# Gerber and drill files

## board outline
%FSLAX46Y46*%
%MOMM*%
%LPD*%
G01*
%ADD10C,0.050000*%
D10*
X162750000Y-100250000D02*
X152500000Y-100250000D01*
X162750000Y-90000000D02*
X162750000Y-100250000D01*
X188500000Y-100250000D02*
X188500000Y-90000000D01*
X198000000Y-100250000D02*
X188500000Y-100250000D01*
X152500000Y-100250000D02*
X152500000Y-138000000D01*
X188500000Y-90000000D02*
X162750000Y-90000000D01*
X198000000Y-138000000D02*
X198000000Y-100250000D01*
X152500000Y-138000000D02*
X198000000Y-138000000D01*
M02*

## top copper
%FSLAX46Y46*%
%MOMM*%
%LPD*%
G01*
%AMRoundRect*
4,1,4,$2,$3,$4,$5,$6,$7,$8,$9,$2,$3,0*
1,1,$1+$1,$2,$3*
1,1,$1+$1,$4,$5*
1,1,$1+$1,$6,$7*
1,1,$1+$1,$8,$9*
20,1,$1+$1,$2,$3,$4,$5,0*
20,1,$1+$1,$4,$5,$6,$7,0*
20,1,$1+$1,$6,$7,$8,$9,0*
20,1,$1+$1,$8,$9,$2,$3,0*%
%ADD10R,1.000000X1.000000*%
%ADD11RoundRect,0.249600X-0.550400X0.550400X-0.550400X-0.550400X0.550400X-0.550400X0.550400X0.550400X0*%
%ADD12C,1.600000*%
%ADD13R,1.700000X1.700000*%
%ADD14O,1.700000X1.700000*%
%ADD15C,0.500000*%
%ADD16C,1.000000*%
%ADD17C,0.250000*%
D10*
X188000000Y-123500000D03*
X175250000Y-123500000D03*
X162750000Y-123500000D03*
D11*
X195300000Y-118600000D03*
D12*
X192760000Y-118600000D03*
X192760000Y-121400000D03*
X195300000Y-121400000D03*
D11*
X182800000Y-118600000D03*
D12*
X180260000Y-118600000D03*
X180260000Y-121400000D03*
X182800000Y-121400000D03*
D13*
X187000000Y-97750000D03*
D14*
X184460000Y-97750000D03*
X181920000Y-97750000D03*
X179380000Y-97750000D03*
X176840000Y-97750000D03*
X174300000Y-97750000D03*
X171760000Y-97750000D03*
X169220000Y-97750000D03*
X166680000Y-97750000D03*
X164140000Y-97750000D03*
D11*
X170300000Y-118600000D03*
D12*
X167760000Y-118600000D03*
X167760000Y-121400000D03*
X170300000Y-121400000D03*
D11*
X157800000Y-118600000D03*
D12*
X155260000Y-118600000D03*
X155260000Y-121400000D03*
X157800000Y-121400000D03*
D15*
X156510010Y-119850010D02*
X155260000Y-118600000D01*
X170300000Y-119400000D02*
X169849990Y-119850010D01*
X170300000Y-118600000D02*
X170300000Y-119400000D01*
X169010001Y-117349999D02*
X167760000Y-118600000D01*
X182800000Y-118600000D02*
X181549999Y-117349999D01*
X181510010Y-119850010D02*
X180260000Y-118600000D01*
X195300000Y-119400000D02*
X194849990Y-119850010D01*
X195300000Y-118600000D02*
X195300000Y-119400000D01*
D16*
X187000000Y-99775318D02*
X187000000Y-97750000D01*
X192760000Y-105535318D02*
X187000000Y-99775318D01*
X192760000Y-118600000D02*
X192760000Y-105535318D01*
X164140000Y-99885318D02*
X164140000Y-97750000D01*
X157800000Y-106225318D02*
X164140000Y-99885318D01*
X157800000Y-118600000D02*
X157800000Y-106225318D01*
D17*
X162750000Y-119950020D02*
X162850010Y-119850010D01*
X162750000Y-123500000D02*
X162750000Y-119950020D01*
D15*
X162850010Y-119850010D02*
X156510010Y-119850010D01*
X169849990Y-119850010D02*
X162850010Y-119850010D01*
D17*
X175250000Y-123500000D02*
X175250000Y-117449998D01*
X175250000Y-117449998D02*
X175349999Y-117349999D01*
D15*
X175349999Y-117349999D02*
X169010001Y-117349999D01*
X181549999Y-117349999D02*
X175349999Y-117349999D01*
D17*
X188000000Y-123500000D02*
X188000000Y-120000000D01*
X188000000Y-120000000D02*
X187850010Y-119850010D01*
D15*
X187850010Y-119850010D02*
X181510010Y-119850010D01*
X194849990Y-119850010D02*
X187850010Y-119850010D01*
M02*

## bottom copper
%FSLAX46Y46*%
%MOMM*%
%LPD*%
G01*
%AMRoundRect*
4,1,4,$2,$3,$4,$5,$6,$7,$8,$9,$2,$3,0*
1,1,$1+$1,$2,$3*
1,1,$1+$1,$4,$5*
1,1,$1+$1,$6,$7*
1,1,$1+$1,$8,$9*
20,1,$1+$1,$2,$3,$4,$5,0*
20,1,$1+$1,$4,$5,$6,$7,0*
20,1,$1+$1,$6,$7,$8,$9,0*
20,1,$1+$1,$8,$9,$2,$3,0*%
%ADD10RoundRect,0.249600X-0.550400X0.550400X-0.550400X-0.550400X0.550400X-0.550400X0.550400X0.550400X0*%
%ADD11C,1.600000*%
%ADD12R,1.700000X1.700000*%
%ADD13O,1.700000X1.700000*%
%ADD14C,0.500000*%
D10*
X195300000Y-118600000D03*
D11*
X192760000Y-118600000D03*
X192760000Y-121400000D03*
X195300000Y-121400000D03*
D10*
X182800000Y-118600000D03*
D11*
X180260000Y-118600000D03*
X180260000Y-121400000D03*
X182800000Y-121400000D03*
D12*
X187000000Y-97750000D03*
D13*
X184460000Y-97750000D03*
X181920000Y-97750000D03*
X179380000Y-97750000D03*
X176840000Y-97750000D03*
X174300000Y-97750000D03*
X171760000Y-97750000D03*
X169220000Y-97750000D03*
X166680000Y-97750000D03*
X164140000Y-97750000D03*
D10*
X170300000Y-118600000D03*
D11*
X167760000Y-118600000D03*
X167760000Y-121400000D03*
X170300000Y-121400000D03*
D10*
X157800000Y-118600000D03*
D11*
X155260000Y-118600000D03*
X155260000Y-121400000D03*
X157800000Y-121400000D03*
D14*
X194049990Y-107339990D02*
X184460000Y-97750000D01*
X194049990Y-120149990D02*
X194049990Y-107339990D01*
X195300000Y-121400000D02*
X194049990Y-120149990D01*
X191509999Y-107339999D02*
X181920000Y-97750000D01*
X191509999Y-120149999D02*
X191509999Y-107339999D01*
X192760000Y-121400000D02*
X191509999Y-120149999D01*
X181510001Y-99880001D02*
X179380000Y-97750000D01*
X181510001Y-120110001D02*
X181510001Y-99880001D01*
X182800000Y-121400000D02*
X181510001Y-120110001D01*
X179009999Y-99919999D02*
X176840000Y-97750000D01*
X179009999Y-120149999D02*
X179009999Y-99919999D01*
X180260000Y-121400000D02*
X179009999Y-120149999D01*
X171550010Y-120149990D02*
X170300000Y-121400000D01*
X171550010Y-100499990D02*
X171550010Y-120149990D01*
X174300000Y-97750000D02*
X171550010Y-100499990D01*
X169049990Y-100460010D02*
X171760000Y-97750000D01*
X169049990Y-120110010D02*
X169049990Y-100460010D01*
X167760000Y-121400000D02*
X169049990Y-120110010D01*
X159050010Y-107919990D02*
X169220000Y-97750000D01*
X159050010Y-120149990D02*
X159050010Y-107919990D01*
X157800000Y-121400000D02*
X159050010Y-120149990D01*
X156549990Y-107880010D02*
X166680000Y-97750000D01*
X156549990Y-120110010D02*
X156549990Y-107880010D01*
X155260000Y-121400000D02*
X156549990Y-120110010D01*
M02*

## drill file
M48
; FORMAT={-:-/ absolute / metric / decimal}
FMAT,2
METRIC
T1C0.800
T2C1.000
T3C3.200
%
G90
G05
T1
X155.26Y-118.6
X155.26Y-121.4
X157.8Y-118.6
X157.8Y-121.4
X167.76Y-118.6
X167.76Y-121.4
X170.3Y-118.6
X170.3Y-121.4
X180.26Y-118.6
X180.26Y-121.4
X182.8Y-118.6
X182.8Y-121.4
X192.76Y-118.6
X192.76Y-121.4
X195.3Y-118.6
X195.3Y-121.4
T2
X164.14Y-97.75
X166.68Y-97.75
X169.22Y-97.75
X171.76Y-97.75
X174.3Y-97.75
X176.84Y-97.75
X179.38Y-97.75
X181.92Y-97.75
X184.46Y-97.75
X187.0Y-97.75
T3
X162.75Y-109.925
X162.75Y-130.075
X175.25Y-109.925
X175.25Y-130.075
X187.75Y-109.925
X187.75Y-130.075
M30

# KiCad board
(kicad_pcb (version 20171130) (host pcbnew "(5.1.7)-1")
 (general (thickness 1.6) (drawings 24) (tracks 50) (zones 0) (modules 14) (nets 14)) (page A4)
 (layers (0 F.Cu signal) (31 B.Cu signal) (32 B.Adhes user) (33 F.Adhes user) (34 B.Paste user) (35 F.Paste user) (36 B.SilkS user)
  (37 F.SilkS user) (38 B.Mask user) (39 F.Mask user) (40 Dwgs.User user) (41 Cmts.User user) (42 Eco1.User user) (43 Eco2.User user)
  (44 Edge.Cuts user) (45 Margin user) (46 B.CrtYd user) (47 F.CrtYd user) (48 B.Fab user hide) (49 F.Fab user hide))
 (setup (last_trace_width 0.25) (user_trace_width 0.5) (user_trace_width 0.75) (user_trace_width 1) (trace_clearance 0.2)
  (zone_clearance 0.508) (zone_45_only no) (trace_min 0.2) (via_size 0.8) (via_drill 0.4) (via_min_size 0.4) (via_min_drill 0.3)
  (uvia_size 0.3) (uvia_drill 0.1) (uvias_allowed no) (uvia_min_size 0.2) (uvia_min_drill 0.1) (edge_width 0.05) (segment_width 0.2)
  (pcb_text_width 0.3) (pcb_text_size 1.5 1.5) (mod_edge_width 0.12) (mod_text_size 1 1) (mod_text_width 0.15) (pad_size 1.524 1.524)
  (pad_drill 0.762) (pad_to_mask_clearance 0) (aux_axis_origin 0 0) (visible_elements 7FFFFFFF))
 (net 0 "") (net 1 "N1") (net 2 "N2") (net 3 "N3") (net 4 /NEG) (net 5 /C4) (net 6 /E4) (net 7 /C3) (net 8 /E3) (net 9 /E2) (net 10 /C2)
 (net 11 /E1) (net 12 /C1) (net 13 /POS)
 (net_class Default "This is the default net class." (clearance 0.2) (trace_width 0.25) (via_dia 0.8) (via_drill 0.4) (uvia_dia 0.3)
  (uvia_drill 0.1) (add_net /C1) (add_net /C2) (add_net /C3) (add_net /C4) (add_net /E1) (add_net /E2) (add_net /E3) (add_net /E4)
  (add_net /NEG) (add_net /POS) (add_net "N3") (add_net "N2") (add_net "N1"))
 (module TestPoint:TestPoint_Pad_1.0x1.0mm (layer F.Cu) (at 188 123.5)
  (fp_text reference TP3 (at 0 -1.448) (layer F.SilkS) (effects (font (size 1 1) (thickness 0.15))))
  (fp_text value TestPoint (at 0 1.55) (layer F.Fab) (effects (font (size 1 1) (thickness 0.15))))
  (pad 1 smd rect (at 0 0) (size 1 1) (layers F.Cu F.Mask) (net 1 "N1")))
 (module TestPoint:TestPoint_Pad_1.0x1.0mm (layer F.Cu) (at 175.25 123.5)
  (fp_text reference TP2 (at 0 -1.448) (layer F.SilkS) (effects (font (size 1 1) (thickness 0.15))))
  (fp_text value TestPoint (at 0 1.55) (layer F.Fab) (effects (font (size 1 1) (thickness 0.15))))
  (pad 1 smd rect (at 0 0) (size 1 1) (layers F.Cu F.Mask) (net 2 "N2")))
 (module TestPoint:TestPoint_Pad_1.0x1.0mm (layer F.Cu) (at 162.75 123.5)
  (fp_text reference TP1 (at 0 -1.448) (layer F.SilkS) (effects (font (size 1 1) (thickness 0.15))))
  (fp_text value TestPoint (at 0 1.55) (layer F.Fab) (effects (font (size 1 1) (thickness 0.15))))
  (pad 1 smd rect (at 0 0) (size 1 1) (layers F.Cu F.Mask) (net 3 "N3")))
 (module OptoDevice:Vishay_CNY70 (layer F.Cu) (at 195.3 118.6 270)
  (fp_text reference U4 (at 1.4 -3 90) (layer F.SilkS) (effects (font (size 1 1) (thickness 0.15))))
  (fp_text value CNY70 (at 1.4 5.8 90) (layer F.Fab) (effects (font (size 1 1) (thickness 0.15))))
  (pad 1 thru_hole roundrect (at 0 0 270) (size 1.6 1.6) (drill 0.8) (layers *.Cu *.Mask) (roundrect_rratio 0.156) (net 1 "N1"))
  (pad 2 thru_hole circle (at 0 2.54 270) (size 1.6 1.6) (drill 0.8) (layers *.Cu *.Mask) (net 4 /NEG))
  (pad 3 thru_hole circle (at 2.8 2.54 270) (size 1.6 1.6) (drill 0.8) (layers *.Cu *.Mask) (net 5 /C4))
  (pad 4 thru_hole circle (at 2.8 0 270) (size 1.6 1.6) (drill 0.8) (layers *.Cu *.Mask) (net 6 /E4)))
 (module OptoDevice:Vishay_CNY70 (layer F.Cu) (at 182.8 118.6 270)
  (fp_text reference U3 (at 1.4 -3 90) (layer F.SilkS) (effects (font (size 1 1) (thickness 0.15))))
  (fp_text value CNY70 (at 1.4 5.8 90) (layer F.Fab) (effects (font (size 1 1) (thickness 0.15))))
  (pad 1 thru_hole roundrect (at 0 0 270) (size 1.6 1.6) (drill 0.8) (layers *.Cu *.Mask) (roundrect_rratio 0.156) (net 2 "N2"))
  (pad 2 thru_hole circle (at 0 2.54 270) (size 1.6 1.6) (drill 0.8) (layers *.Cu *.Mask) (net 1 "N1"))
  (pad 3 thru_hole circle (at 2.8 2.54 270) (size 1.6 1.6) (drill 0.8) (layers *.Cu *.Mask) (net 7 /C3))
  (pad 4 thru_hole circle (at 2.8 0 270) (size 1.6 1.6) (drill 0.8) (layers *.Cu *.Mask) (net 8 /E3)))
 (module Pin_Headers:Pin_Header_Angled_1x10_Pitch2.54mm (layer B.Cu) (at 187 97.75 90)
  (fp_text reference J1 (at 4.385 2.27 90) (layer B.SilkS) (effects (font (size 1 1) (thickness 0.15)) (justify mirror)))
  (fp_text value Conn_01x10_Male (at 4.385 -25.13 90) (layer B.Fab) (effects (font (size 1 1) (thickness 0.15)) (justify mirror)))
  (pad 1 thru_hole rect (at 0 0 90) (size 1.7 1.7) (drill 1) (layers *.Cu *.Mask) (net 4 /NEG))
  (pad 2 thru_hole oval (at 0 -2.54 90) (size 1.7 1.7) (drill 1) (layers *.Cu *.Mask) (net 6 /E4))
  (pad 3 thru_hole oval (at 0 -5.08 90) (size 1.7 1.7) (drill 1) (layers *.Cu *.Mask) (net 5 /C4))
  (pad 4 thru_hole oval (at 0 -7.62 90) (size 1.7 1.7) (drill 1) (layers *.Cu *.Mask) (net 8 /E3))
  (pad 5 thru_hole oval (at 0 -10.16 90) (size 1.7 1.7) (drill 1) (layers *.Cu *.Mask) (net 7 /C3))
  (pad 6 thru_hole oval (at 0 -12.7 90) (size 1.7 1.7) (drill 1) (layers *.Cu *.Mask) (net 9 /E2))
  (pad 7 thru_hole oval (at 0 -15.24 90) (size 1.7 1.7) (drill 1) (layers *.Cu *.Mask) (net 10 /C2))
  (pad 8 thru_hole oval (at 0 -17.78 90) (size 1.7 1.7) (drill 1) (layers *.Cu *.Mask) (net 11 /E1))
  (pad 9 thru_hole oval (at 0 -20.32 90) (size 1.7 1.7) (drill 1) (layers *.Cu *.Mask) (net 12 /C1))
  (pad 10 thru_hole oval (at 0 -22.86 90) (size 1.7 1.7) (drill 1) (layers *.Cu *.Mask) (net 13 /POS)))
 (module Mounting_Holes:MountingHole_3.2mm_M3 (layer F.Cu) (at 187.75 109.925)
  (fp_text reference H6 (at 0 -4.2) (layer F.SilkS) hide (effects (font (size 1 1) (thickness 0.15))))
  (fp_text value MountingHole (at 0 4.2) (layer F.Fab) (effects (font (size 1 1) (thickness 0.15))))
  (pad 1 np_thru_hole circle (at 0 0) (size 3.2 3.2) (drill 3.2) (layers *.Cu *.Mask)))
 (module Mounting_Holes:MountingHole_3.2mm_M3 (layer F.Cu) (at 187.75 130.075)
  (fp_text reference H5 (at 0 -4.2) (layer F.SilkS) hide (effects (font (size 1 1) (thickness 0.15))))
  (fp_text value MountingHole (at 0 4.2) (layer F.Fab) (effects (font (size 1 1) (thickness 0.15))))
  (pad 1 np_thru_hole circle (at 0 0) (size 3.2 3.2) (drill 3.2) (layers *.Cu *.Mask)))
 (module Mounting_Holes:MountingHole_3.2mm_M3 (layer F.Cu) (at 175.25 109.925)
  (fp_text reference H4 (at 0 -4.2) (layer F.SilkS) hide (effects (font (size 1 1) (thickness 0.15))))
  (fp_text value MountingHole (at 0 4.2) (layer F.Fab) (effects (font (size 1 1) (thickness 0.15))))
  (pad 1 np_thru_hole circle (at 0 0) (size 3.2 3.2) (drill 3.2) (layers *.Cu *.Mask)))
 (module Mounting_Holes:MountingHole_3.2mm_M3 (layer F.Cu) (at 175.25 130.075)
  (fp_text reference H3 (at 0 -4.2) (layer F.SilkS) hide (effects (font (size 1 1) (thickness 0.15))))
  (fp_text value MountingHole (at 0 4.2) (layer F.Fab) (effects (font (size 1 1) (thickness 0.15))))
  (pad 1 np_thru_hole circle (at 0 0) (size 3.2 3.2) (drill 3.2) (layers *.Cu *.Mask)))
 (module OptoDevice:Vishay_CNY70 (layer F.Cu) (at 170.3 118.6 270)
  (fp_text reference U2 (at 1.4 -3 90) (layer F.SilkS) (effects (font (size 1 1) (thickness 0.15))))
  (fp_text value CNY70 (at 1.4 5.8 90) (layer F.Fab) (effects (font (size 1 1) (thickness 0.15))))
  (pad 1 thru_hole roundrect (at 0 0 270) (size 1.6 1.6) (drill 0.8) (layers *.Cu *.Mask) (roundrect_rratio 0.156) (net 3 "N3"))
  (pad 2 thru_hole circle (at 0 2.54 270) (size 1.6 1.6) (drill 0.8) (layers *.Cu *.Mask) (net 2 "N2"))
  (pad 3 thru_hole circle (at 2.8 2.54 270) (size 1.6 1.6) (drill 0.8) (layers *.Cu *.Mask) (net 10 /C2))
  (pad 4 thru_hole circle (at 2.8 0 270) (size 1.6 1.6) (drill 0.8) (layers *.Cu *.Mask) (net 9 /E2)))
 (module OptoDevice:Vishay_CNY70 (layer F.Cu) (at 157.8 118.6 270)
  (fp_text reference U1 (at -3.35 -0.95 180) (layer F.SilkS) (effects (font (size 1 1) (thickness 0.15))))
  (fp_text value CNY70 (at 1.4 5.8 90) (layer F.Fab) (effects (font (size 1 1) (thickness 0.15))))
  (pad 1 thru_hole roundrect (at 0 0 270) (size 1.6 1.6) (drill 0.8) (layers *.Cu *.Mask) (roundrect_rratio 0.156) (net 13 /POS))
  (pad 2 thru_hole circle (at 0 2.54 270) (size 1.6 1.6) (drill 0.8) (layers *.Cu *.Mask) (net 3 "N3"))
  (pad 3 thru_hole circle (at 2.8 2.54 270) (size 1.6 1.6) (drill 0.8) (layers *.Cu *.Mask) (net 12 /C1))
  (pad 4 thru_hole circle (at 2.8 0 270) (size 1.6 1.6) (drill 0.8) (layers *.Cu *.Mask) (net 11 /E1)))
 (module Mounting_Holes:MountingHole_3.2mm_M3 (layer F.Cu) (at 162.75 109.925)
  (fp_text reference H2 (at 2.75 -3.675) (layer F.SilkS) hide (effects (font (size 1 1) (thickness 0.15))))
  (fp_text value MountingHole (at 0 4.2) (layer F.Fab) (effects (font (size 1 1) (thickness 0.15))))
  (pad 1 np_thru_hole circle (at 0 0) (size 3.2 3.2) (drill 3.2) (layers *.Cu *.Mask)))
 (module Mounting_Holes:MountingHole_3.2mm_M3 (layer F.Cu) (at 162.75 130.075)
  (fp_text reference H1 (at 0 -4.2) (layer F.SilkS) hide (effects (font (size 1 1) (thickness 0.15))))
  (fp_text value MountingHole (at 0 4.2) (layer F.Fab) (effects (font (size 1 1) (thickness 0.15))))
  (pad 1 np_thru_hole circle (at 0 0) (size 3.2 3.2) (drill 3.2) (layers *.Cu *.Mask)))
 (gr_line (start 162.75 100.25) (end 152.5 100.25) (layer Edge.Cuts) (width 0.05))
 (gr_line (start 162.75 90) (end 162.75 100.25) (layer Edge.Cuts) (width 0.05))
 (gr_line (start 188.5 100.25) (end 188.5 90) (layer Edge.Cuts) (width 0.05))
 (gr_line (start 198 100.25) (end 188.5 100.25) (layer Edge.Cuts) (width 0.05))
 (gr_line (start 152.5 100.25) (end 152.5 138) (layer Edge.Cuts) (width 0.05))
 (gr_line (start 188.5 90) (end 162.75 90) (layer Edge.Cuts) (width 0.05))
 (gr_line (start 198 138) (end 198 100.25) (layer Edge.Cuts) (width 0.05))
 (gr_line (start 152.5 138) (end 198 138) (layer Edge.Cuts) (width 0.05))
 (segment (start 156.51001 119.85001) (end 155.26 118.6) (width 0.5) (layer F.Cu) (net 3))
 (segment (start 170.3 119.4) (end 169.84999 119.85001) (width 0.5) (layer F.Cu) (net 3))
 (segment (start 170.3 118.6) (end 170.3 119.4) (width 0.5) (layer F.Cu) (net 3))
 (segment (start 169.010001 117.349999) (end 167.76 118.6) (width 0.5) (layer F.Cu) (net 2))
 (segment (start 182.8 118.6) (end 181.549999 117.349999) (width 0.5) (layer F.Cu) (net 2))
 (segment (start 181.51001 119.85001) (end 180.26 118.6) (width 0.5) (layer F.Cu) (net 1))
 (segment (start 195.3 119.4) (end 194.84999 119.85001) (width 0.5) (layer F.Cu) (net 1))
 (segment (start 195.3 118.6) (end 195.3 119.4) (width 0.5) (layer F.Cu) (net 1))
 (segment (start 187 99.775318) (end 187 97.75) (width 1) (layer F.Cu) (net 4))
 (segment (start 192.76 105.535318) (end 187 99.775318) (width 1) (layer F.Cu) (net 4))
 (segment (start 192.76 118.6) (end 192.76 105.535318) (width 1) (layer F.Cu) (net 4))
 (segment (start 164.14 99.885318) (end 164.14 97.75) (width 1) (layer F.Cu) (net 13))
 (segment (start 157.8 106.225318) (end 164.14 99.885318) (width 1) (layer F.Cu) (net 13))
 (segment (start 157.8 118.6) (end 157.8 106.225318) (width 1) (layer F.Cu) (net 13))
 (segment (start 194.04999 107.33999) (end 184.46 97.75) (width 0.5) (layer B.Cu) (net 6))
 (segment (start 194.04999 120.14999) (end 194.04999 107.33999) (width 0.5) (layer B.Cu) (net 6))
 (segment (start 195.3 121.4) (end 194.04999 120.14999) (width 0.5) (layer B.Cu) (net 6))
 (segment (start 191.509999 107.339999) (end 181.92 97.75) (width 0.5) (layer B.Cu) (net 5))
 (segment (start 191.509999 120.149999) (end 191.509999 107.339999) (width 0.5) (layer B.Cu) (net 5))
 (segment (start 192.76 121.4) (end 191.509999 120.149999) (width 0.5) (layer B.Cu) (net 5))
 (segment (start 181.510001 99.880001) (end 179.38 97.75) (width 0.5) (layer B.Cu) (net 8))
 (segment (start 181.510001 120.110001) (end 181.510001 99.880001) (width 0.5) (layer B.Cu) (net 8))
 (segment (start 182.8 121.4) (end 181.510001 120.110001) (width 0.5) (layer B.Cu) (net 8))
 (segment (start 179.009999 99.919999) (end 176.84 97.75) (width 0.5) (layer B.Cu) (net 7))
 (segment (start 179.009999 120.149999) (end 179.009999 99.919999) (width 0.5) (layer B.Cu) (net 7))
 (segment (start 180.26 121.4) (end 179.009999 120.149999) (width 0.5) (layer B.Cu) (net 7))
 (segment (start 171.55001 120.14999) (end 170.3 121.4) (width 0.5) (layer B.Cu) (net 9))
 (segment (start 171.55001 100.49999) (end 171.55001 120.14999) (width 0.5) (layer B.Cu) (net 9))
 (segment (start 174.3 97.75) (end 171.55001 100.49999) (width 0.5) (layer B.Cu) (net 9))
 (segment (start 169.04999 100.46001) (end 171.76 97.75) (width 0.5) (layer B.Cu) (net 10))
 (segment (start 169.04999 120.11001) (end 169.04999 100.46001) (width 0.5) (layer B.Cu) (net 10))
 (segment (start 167.76 121.4) (end 169.04999 120.11001) (width 0.5) (layer B.Cu) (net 10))
 (segment (start 159.05001 107.91999) (end 169.22 97.75) (width 0.5) (layer B.Cu) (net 11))
 (segment (start 159.05001 120.14999) (end 159.05001 107.91999) (width 0.5) (layer B.Cu) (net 11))
 (segment (start 157.8 121.4) (end 159.05001 120.14999) (width 0.5) (layer B.Cu) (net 11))
 (segment (start 156.54999 107.88001) (end 166.68 97.75) (width 0.5) (layer B.Cu) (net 12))
 (segment (start 156.54999 120.11001) (end 156.54999 107.88001) (width 0.5) (layer B.Cu) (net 12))
 (segment (start 155.26 121.4) (end 156.54999 120.11001) (width 0.5) (layer B.Cu) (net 12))
 (segment (start 162.75 119.95002) (end 162.85001 119.85001) (width 0.25) (layer F.Cu) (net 3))
 (segment (start 162.75 123.5) (end 162.75 119.95002) (width 0.25) (layer F.Cu) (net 3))
 (segment (start 162.85001 119.85001) (end 156.51001 119.85001) (width 0.5) (layer F.Cu) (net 3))
 (segment (start 169.84999 119.85001) (end 162.85001 119.85001) (width 0.5) (layer F.Cu) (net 3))
 (segment (start 175.25 123.5) (end 175.25 117.449998) (width 0.25) (layer F.Cu) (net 2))
 (segment (start 175.25 117.449998) (end 175.349999 117.349999) (width 0.25) (layer F.Cu) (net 2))
 (segment (start 175.349999 117.349999) (end 169.010001 117.349999) (width 0.5) (layer F.Cu) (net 2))
 (segment (start 181.549999 117.349999) (end 175.349999 117.349999) (width 0.5) (layer F.Cu) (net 2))
 (segment (start 188 123.5) (end 188 120) (width 0.25) (layer F.Cu) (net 1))
 (segment (start 188 120) (end 187.85001 119.85001) (width 0.25) (layer F.Cu) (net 1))
 (segment (start 187.85001 119.85001) (end 181.51001 119.85001) (width 0.5) (layer F.Cu) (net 1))
 (segment (start 194.84999 119.85001) (end 187.85001 119.85001) (width 0.5) (layer F.Cu) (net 1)))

